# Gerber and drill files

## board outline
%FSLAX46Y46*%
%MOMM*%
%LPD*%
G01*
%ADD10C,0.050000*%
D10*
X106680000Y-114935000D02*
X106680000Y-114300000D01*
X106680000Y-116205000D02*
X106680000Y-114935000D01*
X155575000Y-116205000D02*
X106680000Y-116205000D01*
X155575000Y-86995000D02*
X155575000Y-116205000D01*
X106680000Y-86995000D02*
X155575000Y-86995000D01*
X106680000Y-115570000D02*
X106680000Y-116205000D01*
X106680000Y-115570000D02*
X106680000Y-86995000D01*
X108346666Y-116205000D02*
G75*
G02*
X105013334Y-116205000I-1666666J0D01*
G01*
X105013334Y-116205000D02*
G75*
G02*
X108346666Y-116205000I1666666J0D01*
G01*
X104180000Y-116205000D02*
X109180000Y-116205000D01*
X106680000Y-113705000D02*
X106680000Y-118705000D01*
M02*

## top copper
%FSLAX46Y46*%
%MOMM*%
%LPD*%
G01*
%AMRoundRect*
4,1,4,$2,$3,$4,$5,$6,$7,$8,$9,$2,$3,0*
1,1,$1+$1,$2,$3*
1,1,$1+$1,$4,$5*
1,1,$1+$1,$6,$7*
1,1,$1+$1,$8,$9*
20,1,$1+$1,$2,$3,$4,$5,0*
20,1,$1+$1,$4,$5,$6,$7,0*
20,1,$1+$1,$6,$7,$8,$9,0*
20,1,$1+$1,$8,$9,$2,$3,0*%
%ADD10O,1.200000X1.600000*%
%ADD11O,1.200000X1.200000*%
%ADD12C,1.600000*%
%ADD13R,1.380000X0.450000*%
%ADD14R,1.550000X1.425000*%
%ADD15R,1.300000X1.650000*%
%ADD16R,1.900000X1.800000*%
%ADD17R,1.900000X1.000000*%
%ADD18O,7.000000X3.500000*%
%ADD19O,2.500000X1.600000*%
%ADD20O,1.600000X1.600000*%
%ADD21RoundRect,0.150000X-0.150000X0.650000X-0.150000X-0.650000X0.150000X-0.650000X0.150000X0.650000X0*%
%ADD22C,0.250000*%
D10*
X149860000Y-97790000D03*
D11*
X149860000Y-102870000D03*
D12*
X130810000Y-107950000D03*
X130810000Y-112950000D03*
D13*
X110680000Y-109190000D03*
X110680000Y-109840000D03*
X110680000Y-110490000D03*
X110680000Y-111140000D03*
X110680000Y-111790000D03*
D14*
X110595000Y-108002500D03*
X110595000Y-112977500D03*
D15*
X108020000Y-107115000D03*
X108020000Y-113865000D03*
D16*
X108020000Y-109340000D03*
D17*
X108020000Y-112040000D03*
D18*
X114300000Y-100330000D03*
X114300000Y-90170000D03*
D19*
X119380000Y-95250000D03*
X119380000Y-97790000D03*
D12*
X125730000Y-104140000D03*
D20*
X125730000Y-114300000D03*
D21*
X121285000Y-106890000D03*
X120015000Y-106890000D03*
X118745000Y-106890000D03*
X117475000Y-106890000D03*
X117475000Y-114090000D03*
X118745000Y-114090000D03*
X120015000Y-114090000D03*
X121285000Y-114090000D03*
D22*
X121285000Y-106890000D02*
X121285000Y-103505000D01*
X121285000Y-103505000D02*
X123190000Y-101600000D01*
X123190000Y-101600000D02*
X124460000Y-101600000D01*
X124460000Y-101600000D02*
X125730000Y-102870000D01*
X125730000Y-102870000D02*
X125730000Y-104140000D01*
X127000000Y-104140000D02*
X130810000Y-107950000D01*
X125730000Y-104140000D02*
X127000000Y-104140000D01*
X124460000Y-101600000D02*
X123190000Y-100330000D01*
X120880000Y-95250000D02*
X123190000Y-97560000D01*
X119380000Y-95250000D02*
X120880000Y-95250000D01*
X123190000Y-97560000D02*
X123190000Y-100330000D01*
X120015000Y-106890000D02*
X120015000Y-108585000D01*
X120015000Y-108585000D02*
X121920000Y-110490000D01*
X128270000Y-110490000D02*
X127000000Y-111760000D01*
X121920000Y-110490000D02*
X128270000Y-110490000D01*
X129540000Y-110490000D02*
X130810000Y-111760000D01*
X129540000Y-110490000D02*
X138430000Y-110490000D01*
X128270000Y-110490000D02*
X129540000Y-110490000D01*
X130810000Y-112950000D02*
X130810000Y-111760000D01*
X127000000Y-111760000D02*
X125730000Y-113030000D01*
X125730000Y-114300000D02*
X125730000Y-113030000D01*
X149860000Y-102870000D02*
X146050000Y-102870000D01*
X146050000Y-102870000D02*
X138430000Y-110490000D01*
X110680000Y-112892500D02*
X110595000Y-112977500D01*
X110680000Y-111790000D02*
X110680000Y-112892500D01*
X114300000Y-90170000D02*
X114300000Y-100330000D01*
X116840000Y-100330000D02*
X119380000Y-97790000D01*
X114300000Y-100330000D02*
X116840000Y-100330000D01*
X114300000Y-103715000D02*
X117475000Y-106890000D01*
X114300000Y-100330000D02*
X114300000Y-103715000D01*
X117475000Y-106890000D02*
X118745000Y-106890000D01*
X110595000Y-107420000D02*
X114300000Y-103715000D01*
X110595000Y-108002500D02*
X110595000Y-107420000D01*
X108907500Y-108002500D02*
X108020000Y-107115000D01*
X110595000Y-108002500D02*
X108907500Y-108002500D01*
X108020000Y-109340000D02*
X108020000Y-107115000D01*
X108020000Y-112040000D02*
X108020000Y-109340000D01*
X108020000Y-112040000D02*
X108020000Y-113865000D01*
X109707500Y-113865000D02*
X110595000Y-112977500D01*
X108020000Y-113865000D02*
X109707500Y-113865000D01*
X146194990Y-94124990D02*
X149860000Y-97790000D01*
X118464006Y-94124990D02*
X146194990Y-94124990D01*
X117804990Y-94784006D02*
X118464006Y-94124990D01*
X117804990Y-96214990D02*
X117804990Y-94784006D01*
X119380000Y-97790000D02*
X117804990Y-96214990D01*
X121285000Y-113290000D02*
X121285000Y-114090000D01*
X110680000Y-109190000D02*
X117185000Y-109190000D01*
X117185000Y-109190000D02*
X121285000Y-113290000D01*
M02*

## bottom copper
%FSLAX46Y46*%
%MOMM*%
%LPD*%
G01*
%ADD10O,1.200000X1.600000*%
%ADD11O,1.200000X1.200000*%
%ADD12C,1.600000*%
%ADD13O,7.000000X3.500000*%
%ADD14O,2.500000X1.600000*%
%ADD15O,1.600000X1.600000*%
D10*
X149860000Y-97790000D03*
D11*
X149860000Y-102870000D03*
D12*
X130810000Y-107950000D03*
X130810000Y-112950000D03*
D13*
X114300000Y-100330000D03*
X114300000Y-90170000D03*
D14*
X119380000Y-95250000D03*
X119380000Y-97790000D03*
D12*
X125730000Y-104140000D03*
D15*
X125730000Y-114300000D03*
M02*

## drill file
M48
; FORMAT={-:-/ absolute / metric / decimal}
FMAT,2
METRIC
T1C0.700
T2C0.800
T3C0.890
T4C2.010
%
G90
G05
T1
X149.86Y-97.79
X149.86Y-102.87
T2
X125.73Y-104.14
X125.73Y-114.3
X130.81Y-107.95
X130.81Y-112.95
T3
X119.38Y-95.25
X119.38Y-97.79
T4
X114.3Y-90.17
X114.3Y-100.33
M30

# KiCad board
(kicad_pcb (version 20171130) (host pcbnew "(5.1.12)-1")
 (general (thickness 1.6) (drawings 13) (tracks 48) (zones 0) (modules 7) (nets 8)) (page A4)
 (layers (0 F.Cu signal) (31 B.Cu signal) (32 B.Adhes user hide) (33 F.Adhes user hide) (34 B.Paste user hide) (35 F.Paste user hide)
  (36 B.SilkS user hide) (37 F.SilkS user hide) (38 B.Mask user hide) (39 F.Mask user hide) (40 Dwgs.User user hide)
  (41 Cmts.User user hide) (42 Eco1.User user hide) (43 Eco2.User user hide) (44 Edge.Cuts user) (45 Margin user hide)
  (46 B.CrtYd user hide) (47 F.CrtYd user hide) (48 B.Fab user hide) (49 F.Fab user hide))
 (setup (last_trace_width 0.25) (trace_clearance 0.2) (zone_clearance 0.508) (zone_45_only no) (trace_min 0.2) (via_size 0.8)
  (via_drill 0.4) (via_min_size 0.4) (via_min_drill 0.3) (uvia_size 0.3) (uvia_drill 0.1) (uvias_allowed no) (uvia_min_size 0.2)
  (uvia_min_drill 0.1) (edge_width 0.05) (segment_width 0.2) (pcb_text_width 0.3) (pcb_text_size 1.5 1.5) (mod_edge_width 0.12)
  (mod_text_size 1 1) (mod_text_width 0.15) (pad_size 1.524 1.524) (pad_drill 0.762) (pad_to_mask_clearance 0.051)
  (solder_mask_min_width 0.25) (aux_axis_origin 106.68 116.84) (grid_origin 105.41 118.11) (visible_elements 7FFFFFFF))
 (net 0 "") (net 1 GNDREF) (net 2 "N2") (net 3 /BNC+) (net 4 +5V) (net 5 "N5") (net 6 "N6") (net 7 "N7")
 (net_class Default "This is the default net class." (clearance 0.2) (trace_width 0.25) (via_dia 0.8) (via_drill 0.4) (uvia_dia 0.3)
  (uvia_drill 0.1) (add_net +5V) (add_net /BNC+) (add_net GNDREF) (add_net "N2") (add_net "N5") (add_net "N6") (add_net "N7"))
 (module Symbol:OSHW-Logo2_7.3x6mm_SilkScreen (layer F.Cu) (at 151.13 90.805)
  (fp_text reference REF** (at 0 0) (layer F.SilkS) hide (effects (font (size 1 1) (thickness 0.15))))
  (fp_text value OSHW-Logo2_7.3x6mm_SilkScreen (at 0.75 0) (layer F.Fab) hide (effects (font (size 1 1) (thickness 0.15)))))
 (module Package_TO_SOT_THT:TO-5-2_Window (layer F.Cu) (at 149.86 97.79 270)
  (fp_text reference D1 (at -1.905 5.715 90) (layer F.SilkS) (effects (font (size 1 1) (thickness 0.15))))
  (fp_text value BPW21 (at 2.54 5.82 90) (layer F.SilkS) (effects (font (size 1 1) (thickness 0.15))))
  (pad 1 thru_hole oval (at 0 0 270) (size 1.6 1.2) (drill 0.7) (layers *.Cu *.Mask) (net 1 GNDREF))
  (pad 2 thru_hole oval (at 5.08 0 270) (size 1.2 1.2) (drill 0.7) (layers *.Cu *.Mask) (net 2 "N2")))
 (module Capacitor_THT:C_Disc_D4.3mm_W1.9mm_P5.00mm (layer F.Cu) (at 130.81 107.95 270)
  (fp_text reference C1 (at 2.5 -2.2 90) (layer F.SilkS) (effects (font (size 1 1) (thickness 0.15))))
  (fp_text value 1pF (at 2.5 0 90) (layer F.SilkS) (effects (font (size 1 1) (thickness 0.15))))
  (pad 1 thru_hole circle (at 0 0 270) (size 1.6 1.6) (drill 0.8) (layers *.Cu *.Mask) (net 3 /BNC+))
  (pad 2 thru_hole circle (at 5 0 270) (size 1.6 1.6) (drill 0.8) (layers *.Cu *.Mask) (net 2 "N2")))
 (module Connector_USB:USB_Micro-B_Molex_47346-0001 (layer F.Cu) (at 109.22 110.49 270)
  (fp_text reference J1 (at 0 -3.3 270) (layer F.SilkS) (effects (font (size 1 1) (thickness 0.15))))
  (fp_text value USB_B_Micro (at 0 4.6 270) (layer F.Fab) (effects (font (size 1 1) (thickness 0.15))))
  (pad 1 smd rect (at -1.3 -1.46 270) (size 0.45 1.38) (layers F.Cu F.Paste F.Mask) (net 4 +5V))
  (pad 2 smd rect (at -0.65 -1.46 270) (size 0.45 1.38) (layers F.Cu F.Paste F.Mask) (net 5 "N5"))
  (pad 3 smd rect (at 0 -1.46 270) (size 0.45 1.38) (layers F.Cu F.Paste F.Mask) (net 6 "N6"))
  (pad 4 smd rect (at 0.65 -1.46 270) (size 0.45 1.38) (layers F.Cu F.Paste F.Mask) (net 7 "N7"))
  (pad 5 smd rect (at 1.3 -1.46 270) (size 0.45 1.38) (layers F.Cu F.Paste F.Mask) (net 1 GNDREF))
  (pad 6 smd rect (at -2.4875 -1.375 270) (size 1.425 1.55) (layers F.Cu F.Paste F.Mask) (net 1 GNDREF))
  (pad 6 smd rect (at 2.4875 -1.375 270) (size 1.425 1.55) (layers F.Cu F.Paste F.Mask) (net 1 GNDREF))
  (pad 6 smd rect (at -3.375 1.2 270) (size 1.65 1.3) (layers F.Cu F.Paste F.Mask) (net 1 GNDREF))
  (pad 6 smd rect (at 3.375 1.2 270) (size 1.65 1.3) (layers F.Cu F.Paste F.Mask) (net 1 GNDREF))
  (pad 6 smd rect (at -1.15 1.2 270) (size 1.8 1.9) (layers F.Cu F.Paste F.Mask) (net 1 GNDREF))
  (pad 6 smd rect (at 1.55 1.2 270) (size 1 1.9) (layers F.Cu F.Paste F.Mask) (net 1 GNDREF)))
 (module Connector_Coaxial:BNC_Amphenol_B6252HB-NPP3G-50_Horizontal (layer F.Cu) (at 119.38 95.25 90)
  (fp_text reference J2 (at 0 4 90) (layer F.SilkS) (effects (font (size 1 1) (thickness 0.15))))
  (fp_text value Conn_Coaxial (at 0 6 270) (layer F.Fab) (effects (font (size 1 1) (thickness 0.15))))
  (pad 2 thru_hole oval (at -5.08 -5.08 90) (size 3.5 7) (drill 2.01) (layers *.Cu *.Mask) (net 1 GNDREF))
  (pad 2 thru_hole oval (at 5.08 -5.08 90) (size 3.5 7) (drill 2.01) (layers *.Cu *.Mask) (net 1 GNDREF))
  (pad 1 thru_hole oval (at 0 0 90) (size 1.6 2.5) (drill 0.89) (layers *.Cu *.Mask) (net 3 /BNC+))
  (pad 2 thru_hole oval (at -2.54 0 90) (size 1.6 2.5) (drill 0.89) (layers *.Cu *.Mask) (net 1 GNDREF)))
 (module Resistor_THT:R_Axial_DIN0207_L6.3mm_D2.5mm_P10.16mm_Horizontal (layer F.Cu) (at 125.73 104.14 270)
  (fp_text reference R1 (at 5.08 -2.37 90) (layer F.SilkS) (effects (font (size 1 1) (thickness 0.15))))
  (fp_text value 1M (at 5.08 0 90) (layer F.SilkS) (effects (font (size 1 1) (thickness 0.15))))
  (pad 1 thru_hole circle (at 0 0 270) (size 1.6 1.6) (drill 0.8) (layers *.Cu *.Mask) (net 3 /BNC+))
  (pad 2 thru_hole oval (at 10.16 0 270) (size 1.6 1.6) (drill 0.8) (layers *.Cu *.Mask) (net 2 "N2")))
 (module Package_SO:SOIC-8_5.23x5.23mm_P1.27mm (layer F.Cu) (at 119.38 110.49 270)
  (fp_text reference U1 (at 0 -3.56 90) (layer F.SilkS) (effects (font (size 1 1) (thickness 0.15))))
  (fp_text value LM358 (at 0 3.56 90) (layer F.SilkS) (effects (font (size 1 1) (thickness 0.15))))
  (pad 1 smd roundrect (at -3.6 -1.905 270) (size 1.6 0.6) (layers F.Cu F.Paste F.Mask) (roundrect_rratio 0.25) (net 3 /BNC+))
  (pad 2 smd roundrect (at -3.6 -0.635 270) (size 1.6 0.6) (layers F.Cu F.Paste F.Mask) (roundrect_rratio 0.25) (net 2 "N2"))
  (pad 3 smd roundrect (at -3.6 0.635 270) (size 1.6 0.6) (layers F.Cu F.Paste F.Mask) (roundrect_rratio 0.25) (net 1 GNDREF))
  (pad 4 smd roundrect (at -3.6 1.905 270) (size 1.6 0.6) (layers F.Cu F.Paste F.Mask) (roundrect_rratio 0.25) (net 1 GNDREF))
  (pad 5 smd roundrect (at 3.6 1.905 270) (size 1.6 0.6) (layers F.Cu F.Paste F.Mask) (roundrect_rratio 0.25))
  (pad 6 smd roundrect (at 3.6 0.635 270) (size 1.6 0.6) (layers F.Cu F.Paste F.Mask) (roundrect_rratio 0.25))
  (pad 7 smd roundrect (at 3.6 -0.635 270) (size 1.6 0.6) (layers F.Cu F.Paste F.Mask) (roundrect_rratio 0.25))
  (pad 8 smd roundrect (at 3.6 -1.905 270) (size 1.6 0.6) (layers F.Cu F.Paste F.Mask) (roundrect_rratio 0.25) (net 4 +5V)))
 (gr_line (start 106.68 114.935) (end 106.68 114.3) (layer Edge.Cuts) (width 0.05))
 (gr_line (start 106.68 116.205) (end 106.68 114.935) (layer Edge.Cuts) (width 0.05))
 (gr_line (start 155.575 116.205) (end 106.68 116.205) (layer Edge.Cuts) (width 0.05))
 (gr_line (start 155.575 86.995) (end 155.575 116.205) (layer Edge.Cuts) (width 0.05))
 (gr_line (start 106.68 86.995) (end 155.575 86.995) (layer Edge.Cuts) (width 0.05))
 (gr_line (start 106.68 115.57) (end 106.68 116.205) (layer Edge.Cuts) (width 0.05))
 (gr_line (start 106.68 115.57) (end 106.68 86.995) (layer Edge.Cuts) (width 0.05))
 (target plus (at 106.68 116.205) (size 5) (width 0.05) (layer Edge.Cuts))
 (segment (start 121.285 106.89) (end 121.285 103.505) (width 0.25) (layer F.Cu) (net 3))
 (segment (start 121.285 103.505) (end 123.19 101.6) (width 0.25) (layer F.Cu) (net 3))
 (segment (start 123.19 101.6) (end 124.46 101.6) (width 0.25) (layer F.Cu) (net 3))
 (segment (start 124.46 101.6) (end 125.73 102.87) (width 0.25) (layer F.Cu) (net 3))
 (segment (start 125.73 102.87) (end 125.73 104.14) (width 0.25) (layer F.Cu) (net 3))
 (segment (start 127 104.14) (end 130.81 107.95) (width 0.25) (layer F.Cu) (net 3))
 (segment (start 125.73 104.14) (end 127 104.14) (width 0.25) (layer F.Cu) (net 3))
 (segment (start 124.46 101.6) (end 123.19 100.33) (width 0.25) (layer F.Cu) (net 3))
 (segment (start 120.88 95.25) (end 123.19 97.56) (width 0.25) (layer F.Cu) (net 3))
 (segment (start 119.38 95.25) (end 120.88 95.25) (width 0.25) (layer F.Cu) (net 3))
 (segment (start 123.19 97.56) (end 123.19 100.33) (width 0.25) (layer F.Cu) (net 3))
 (segment (start 120.015 106.89) (end 120.015 108.585) (width 0.25) (layer F.Cu) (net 2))
 (segment (start 120.015 108.585) (end 121.92 110.49) (width 0.25) (layer F.Cu) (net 2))
 (segment (start 128.27 110.49) (end 127 111.76) (width 0.25) (layer F.Cu) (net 2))
 (segment (start 121.92 110.49) (end 128.27 110.49) (width 0.25) (layer F.Cu) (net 2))
 (segment (start 129.54 110.49) (end 130.81 111.76) (width 0.25) (layer F.Cu) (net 2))
 (segment (start 129.54 110.49) (end 138.43 110.49) (width 0.25) (layer F.Cu) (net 2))
 (segment (start 128.27 110.49) (end 129.54 110.49) (width 0.25) (layer F.Cu) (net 2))
 (segment (start 130.81 112.95) (end 130.81 111.76) (width 0.25) (layer F.Cu) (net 2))
 (segment (start 127 111.76) (end 125.73 113.03) (width 0.25) (layer F.Cu) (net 2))
 (segment (start 125.73 114.3) (end 125.73 113.03) (width 0.25) (layer F.Cu) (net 2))
 (segment (start 149.86 102.87) (end 146.05 102.87) (width 0.25) (layer F.Cu) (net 2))
 (segment (start 146.05 102.87) (end 138.43 110.49) (width 0.25) (layer F.Cu) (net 2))
 (segment (start 110.68 112.8925) (end 110.595 112.9775) (width 0.25) (layer F.Cu) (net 1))
 (segment (start 110.68 111.79) (end 110.68 112.8925) (width 0.25) (layer F.Cu) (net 1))
 (segment (start 114.3 90.17) (end 114.3 100.33) (width 0.25) (layer F.Cu) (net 1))
 (segment (start 116.84 100.33) (end 119.38 97.79) (width 0.25) (layer F.Cu) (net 1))
 (segment (start 114.3 100.33) (end 116.84 100.33) (width 0.25) (layer F.Cu) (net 1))
 (segment (start 114.3 103.715) (end 117.475 106.89) (width 0.25) (layer F.Cu) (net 1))
 (segment (start 114.3 100.33) (end 114.3 103.715) (width 0.25) (layer F.Cu) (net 1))
 (segment (start 117.475 106.89) (end 118.745 106.89) (width 0.25) (layer F.Cu) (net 1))
 (segment (start 110.595 107.42) (end 114.3 103.715) (width 0.25) (layer F.Cu) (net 1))
 (segment (start 110.595 108.0025) (end 110.595 107.42) (width 0.25) (layer F.Cu) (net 1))
 (segment (start 108.9075 108.0025) (end 108.02 107.115) (width 0.25) (layer F.Cu) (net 1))
 (segment (start 110.595 108.0025) (end 108.9075 108.0025) (width 0.25) (layer F.Cu) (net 1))
 (segment (start 108.02 109.34) (end 108.02 107.115) (width 0.25) (layer F.Cu) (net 1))
 (segment (start 108.02 112.04) (end 108.02 109.34) (width 0.25) (layer F.Cu) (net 1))
 (segment (start 108.02 112.04) (end 108.02 113.865) (width 0.25) (layer F.Cu) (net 1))
 (segment (start 109.7075 113.865) (end 110.595 112.9775) (width 0.25) (layer F.Cu) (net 1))
 (segment (start 108.02 113.865) (end 109.7075 113.865) (width 0.25) (layer F.Cu) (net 1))
 (segment (start 146.19499 94.12499) (end 149.86 97.79) (width 0.25) (layer F.Cu) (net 1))
 (segment (start 118.464006 94.12499) (end 146.19499 94.12499) (width 0.25) (layer F.Cu) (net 1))
 (segment (start 117.80499 94.784006) (end 118.464006 94.12499) (width 0.25) (layer F.Cu) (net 1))
 (segment (start 117.80499 96.21499) (end 117.80499 94.784006) (width 0.25) (layer F.Cu) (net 1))
 (segment (start 119.38 97.79) (end 117.80499 96.21499) (width 0.25) (layer F.Cu) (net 1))
 (segment (start 121.285 113.29) (end 121.285 114.09) (width 0.25) (layer F.Cu) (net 4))
 (segment (start 110.68 109.19) (end 117.185 109.19) (width 0.25) (layer F.Cu) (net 4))
 (segment (start 117.185 109.19) (end 121.285 113.29) (width 0.25) (layer F.Cu) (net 4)))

